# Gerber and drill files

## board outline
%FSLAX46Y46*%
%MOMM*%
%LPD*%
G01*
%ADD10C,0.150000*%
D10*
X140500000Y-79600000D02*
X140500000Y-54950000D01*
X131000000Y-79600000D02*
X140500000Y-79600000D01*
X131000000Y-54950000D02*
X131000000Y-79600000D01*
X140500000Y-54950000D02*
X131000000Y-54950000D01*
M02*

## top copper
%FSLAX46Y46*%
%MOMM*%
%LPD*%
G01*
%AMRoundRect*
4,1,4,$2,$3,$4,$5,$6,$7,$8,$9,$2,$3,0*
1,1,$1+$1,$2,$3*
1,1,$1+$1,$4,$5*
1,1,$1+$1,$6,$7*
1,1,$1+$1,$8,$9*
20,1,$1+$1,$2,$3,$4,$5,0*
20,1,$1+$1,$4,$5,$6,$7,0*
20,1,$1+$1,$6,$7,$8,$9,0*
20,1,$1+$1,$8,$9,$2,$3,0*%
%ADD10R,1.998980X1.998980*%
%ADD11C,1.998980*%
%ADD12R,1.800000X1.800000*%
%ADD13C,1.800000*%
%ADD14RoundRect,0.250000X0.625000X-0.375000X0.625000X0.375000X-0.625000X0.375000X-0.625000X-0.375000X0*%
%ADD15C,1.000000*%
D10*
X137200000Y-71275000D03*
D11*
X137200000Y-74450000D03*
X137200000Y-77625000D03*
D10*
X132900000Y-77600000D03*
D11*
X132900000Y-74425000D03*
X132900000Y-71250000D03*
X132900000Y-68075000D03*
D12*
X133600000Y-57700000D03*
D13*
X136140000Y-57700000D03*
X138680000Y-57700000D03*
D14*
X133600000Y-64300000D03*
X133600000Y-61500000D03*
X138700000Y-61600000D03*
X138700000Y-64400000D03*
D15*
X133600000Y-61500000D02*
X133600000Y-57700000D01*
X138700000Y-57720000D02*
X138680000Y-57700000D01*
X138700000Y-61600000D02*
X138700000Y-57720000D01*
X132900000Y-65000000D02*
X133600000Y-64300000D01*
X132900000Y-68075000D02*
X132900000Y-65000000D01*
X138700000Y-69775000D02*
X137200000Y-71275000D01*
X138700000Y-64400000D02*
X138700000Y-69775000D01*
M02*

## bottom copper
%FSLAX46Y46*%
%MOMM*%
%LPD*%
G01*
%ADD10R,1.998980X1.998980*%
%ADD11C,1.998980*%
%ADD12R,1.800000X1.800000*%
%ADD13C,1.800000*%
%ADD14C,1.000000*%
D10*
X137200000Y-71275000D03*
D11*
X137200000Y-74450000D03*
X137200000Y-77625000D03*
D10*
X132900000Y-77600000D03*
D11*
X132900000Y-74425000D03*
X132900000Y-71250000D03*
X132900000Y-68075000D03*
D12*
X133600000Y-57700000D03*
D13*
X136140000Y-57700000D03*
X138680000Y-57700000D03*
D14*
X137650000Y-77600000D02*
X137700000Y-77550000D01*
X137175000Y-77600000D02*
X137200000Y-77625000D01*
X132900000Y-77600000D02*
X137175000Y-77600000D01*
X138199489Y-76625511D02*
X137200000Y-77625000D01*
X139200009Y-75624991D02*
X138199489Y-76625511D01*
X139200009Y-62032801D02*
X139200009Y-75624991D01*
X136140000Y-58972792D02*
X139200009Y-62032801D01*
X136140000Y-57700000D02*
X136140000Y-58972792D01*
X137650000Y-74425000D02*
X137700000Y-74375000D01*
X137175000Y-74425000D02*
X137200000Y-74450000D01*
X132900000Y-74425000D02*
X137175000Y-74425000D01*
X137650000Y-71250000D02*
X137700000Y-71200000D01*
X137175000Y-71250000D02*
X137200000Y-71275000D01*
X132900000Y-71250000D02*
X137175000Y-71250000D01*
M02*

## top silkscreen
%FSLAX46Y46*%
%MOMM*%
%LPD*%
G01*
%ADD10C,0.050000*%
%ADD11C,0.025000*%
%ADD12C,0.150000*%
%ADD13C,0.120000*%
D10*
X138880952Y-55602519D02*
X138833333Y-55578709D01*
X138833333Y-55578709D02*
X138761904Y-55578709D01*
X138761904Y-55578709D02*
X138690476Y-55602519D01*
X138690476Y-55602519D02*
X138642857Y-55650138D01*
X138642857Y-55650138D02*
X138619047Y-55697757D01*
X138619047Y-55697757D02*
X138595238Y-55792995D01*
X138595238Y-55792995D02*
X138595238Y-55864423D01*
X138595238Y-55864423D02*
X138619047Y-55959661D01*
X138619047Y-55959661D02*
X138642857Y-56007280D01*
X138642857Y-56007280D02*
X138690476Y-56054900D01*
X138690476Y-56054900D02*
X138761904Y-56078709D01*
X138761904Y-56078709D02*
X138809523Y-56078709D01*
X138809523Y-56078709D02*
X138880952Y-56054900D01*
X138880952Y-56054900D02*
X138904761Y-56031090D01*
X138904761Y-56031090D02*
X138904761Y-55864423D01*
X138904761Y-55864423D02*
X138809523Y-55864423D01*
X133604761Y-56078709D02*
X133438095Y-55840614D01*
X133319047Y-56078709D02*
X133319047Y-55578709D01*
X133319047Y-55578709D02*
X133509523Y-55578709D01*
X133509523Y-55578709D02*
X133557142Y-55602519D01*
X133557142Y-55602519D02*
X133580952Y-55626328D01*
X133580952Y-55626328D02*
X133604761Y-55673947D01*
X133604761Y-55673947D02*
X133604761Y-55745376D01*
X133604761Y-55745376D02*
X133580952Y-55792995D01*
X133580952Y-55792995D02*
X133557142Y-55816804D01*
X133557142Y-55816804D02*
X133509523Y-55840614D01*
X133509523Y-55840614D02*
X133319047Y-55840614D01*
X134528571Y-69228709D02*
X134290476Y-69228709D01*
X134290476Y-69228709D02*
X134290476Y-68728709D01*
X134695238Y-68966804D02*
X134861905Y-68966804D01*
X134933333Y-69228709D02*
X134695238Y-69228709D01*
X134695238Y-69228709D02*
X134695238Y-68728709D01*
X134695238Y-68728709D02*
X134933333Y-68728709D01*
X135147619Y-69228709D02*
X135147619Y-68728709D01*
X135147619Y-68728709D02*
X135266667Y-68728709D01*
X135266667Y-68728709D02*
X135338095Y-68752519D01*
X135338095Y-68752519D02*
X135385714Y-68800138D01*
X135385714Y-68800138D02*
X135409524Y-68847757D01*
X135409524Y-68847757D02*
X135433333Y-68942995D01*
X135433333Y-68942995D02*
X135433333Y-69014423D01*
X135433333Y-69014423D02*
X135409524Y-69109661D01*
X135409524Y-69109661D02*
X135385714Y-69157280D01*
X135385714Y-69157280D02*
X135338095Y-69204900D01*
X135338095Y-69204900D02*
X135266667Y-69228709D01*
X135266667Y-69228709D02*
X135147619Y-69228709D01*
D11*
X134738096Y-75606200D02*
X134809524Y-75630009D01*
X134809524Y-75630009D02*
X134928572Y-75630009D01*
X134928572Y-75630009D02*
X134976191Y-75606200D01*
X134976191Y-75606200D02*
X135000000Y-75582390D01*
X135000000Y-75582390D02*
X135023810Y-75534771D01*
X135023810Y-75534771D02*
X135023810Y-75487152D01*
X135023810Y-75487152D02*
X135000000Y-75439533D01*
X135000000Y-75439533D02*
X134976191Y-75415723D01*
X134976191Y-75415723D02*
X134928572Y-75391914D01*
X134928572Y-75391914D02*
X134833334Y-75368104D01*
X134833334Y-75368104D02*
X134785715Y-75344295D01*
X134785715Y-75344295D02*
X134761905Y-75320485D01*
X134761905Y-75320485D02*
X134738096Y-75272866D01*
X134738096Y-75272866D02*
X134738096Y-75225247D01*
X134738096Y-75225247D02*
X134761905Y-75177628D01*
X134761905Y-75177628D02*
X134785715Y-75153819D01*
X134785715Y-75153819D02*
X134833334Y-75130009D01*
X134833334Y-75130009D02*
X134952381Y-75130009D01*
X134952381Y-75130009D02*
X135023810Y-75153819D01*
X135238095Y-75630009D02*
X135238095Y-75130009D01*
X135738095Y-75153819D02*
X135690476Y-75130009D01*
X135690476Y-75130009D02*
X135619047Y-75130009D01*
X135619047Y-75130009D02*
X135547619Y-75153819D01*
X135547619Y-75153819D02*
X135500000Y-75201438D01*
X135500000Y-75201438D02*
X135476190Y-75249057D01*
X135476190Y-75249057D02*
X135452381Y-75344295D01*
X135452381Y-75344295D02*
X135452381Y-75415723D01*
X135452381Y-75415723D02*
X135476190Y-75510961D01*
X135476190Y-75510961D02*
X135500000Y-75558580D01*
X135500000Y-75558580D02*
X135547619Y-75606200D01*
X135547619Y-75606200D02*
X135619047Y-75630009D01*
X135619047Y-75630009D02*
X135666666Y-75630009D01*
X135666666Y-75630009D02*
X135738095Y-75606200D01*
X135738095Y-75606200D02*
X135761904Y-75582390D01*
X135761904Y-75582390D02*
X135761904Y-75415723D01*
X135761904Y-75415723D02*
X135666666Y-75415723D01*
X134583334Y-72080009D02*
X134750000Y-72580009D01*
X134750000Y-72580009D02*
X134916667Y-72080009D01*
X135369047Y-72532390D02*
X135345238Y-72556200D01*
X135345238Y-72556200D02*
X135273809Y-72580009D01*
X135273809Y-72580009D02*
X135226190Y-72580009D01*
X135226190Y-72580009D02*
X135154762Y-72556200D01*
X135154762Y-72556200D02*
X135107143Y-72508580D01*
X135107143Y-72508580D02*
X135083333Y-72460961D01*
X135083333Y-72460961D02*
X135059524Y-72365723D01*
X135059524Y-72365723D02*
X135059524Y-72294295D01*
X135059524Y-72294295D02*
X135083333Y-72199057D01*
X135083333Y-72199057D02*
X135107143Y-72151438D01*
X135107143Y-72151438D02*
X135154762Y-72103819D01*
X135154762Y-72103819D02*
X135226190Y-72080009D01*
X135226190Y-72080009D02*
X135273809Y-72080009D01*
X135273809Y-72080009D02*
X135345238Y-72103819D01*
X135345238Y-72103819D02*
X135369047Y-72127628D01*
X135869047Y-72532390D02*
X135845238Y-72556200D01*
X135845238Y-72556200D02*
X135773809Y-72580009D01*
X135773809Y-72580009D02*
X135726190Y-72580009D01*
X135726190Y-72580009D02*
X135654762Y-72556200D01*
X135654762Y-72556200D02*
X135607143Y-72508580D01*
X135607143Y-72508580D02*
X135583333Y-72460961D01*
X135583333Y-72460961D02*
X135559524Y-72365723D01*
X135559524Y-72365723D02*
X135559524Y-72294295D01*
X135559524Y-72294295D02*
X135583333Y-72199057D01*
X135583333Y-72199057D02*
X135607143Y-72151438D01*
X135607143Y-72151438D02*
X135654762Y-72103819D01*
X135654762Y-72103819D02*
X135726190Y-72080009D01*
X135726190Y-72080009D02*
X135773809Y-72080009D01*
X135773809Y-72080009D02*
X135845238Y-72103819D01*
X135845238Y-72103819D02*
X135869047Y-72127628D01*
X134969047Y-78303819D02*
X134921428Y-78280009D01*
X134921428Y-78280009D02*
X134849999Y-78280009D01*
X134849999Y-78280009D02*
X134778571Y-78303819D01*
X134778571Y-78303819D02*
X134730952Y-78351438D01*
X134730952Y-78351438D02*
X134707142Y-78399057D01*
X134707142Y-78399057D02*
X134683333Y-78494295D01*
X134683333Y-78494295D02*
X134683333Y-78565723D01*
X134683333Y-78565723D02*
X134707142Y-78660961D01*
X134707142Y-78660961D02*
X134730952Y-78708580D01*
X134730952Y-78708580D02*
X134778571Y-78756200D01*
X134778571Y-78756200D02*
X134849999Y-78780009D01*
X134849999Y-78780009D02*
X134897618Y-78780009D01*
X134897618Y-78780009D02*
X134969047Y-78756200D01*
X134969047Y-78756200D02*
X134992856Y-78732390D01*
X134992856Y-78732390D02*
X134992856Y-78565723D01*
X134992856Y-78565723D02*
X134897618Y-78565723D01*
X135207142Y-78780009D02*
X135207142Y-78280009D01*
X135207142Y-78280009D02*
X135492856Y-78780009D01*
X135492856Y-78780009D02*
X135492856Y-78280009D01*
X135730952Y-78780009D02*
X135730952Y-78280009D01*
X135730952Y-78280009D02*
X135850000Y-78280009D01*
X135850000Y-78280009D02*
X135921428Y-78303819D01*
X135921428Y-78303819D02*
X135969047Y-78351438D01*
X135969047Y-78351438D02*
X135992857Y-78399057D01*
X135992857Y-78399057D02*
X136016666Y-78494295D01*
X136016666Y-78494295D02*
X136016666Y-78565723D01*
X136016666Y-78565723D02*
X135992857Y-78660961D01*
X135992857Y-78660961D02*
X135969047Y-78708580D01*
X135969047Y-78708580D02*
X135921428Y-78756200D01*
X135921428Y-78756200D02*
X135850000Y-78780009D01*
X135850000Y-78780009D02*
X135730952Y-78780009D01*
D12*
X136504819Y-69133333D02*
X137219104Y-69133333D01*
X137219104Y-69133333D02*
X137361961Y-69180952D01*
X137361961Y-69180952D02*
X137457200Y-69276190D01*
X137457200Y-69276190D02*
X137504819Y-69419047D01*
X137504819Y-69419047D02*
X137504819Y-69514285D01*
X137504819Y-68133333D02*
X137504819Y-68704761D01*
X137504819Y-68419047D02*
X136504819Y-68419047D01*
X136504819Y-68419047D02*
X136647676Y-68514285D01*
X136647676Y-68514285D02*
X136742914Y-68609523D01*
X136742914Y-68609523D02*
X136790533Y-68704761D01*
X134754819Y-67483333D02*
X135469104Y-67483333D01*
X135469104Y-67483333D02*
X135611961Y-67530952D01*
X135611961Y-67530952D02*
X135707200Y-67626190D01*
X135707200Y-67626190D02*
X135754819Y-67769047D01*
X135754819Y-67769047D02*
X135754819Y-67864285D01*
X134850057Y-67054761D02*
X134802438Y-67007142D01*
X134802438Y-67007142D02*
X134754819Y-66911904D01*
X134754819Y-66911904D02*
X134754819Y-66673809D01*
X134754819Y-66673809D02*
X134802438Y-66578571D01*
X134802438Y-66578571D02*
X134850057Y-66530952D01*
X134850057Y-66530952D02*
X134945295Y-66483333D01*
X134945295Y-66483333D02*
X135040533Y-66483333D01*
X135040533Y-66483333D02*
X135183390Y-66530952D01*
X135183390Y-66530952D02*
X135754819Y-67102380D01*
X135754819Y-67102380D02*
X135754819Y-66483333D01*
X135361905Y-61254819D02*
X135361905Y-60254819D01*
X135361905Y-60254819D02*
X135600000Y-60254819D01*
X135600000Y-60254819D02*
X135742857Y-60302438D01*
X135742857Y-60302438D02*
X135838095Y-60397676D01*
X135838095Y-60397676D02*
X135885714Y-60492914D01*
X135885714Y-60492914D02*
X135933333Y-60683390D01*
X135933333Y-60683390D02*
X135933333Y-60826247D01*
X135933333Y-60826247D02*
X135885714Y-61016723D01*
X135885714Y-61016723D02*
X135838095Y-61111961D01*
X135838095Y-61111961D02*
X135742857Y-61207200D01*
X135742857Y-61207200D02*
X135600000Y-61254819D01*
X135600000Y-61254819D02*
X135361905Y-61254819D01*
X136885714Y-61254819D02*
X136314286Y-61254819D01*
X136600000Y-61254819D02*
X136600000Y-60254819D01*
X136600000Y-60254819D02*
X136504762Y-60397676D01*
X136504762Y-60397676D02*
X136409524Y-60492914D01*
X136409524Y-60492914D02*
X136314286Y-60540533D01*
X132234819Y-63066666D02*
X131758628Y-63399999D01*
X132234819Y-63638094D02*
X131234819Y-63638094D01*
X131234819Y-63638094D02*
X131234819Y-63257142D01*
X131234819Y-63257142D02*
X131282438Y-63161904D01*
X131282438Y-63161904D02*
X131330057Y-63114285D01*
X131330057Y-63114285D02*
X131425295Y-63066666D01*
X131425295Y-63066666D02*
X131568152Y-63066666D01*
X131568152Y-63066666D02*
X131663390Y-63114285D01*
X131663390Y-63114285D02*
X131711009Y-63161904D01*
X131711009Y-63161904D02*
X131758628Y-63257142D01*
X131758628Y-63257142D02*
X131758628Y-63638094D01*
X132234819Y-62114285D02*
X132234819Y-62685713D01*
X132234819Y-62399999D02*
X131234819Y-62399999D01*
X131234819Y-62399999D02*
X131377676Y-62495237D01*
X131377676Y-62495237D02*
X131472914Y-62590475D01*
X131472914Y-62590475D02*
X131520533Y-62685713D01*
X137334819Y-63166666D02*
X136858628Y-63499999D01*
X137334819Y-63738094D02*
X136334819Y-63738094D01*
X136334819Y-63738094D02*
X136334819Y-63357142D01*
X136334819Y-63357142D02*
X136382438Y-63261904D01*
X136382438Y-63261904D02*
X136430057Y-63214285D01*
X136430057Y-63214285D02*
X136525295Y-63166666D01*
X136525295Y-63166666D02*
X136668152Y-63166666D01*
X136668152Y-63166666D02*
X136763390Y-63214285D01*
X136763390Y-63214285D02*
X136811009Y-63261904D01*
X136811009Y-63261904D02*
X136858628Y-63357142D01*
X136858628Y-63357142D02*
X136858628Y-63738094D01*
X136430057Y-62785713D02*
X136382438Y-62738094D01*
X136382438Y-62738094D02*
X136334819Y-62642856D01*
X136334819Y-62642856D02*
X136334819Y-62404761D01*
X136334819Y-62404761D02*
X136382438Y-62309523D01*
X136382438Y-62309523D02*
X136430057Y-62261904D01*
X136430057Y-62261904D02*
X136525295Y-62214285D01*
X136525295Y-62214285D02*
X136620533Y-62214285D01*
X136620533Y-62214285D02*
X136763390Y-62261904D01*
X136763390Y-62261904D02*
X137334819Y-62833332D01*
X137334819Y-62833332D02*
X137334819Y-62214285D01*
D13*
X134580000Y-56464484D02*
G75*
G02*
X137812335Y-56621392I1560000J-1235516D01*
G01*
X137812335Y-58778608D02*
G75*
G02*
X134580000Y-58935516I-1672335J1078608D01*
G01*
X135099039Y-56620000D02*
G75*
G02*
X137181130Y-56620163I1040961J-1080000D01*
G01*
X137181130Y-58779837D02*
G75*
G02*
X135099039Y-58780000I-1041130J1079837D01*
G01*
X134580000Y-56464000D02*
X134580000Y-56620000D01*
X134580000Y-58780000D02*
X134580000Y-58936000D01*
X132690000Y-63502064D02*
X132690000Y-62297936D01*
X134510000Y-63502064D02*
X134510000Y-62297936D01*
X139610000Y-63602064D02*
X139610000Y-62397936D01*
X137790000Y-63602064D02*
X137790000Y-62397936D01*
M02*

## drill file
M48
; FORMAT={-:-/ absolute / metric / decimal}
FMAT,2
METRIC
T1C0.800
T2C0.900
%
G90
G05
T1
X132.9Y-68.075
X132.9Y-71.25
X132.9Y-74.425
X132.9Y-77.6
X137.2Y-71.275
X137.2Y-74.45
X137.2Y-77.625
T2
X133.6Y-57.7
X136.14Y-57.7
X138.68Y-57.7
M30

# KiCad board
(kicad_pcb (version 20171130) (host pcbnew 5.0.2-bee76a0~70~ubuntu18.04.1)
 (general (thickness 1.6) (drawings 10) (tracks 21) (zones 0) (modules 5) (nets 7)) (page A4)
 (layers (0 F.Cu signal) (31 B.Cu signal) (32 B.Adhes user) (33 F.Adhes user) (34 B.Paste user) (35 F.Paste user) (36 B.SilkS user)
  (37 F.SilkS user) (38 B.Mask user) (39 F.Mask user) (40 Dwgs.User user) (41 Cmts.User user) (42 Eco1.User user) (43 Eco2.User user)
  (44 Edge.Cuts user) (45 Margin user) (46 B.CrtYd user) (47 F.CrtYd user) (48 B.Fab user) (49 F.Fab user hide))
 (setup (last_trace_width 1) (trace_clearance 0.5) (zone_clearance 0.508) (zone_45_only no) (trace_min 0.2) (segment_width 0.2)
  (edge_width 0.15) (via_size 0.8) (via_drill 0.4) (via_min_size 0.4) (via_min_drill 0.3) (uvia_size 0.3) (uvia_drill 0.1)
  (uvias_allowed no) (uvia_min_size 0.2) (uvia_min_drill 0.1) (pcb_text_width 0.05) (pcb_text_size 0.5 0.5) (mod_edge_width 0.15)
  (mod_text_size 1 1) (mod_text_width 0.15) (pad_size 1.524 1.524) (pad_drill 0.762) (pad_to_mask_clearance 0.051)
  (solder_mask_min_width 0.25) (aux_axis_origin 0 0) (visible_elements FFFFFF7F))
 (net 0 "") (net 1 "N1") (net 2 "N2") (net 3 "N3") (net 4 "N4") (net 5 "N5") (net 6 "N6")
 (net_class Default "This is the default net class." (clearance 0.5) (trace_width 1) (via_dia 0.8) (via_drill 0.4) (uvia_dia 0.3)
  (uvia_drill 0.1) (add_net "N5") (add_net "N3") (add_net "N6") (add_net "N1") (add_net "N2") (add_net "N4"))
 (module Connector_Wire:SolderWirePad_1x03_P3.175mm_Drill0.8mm (layer F.Cu) (at 137.2 71.275 270)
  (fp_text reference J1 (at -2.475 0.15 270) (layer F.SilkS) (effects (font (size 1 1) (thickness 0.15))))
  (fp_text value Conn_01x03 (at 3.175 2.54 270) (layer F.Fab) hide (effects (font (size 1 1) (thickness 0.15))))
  (pad 1 thru_hole rect (at 0 0 270) (size 1.99898 1.99898) (drill 0.8001) (layers *.Cu *.Mask) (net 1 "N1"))
  (pad 2 thru_hole circle (at 3.175 0 270) (size 1.99898 1.99898) (drill 0.8001) (layers *.Cu *.Mask) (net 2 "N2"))
  (pad 3 thru_hole circle (at 6.35 0 270) (size 1.99898 1.99898) (drill 0.8001) (layers *.Cu *.Mask) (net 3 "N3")))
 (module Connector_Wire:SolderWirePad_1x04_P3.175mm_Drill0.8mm (layer F.Cu) (at 132.9 77.6 90)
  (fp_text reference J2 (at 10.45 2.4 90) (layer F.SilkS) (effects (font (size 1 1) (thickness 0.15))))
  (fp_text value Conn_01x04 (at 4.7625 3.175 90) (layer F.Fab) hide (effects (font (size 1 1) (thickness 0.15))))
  (pad 1 thru_hole rect (at 0 0 90) (size 1.99898 1.99898) (drill 0.8001) (layers *.Cu *.Mask) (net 3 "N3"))
  (pad 2 thru_hole circle (at 3.175 0 90) (size 1.99898 1.99898) (drill 0.8001) (layers *.Cu *.Mask) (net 2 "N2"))
  (pad 3 thru_hole circle (at 6.35 0 90) (size 1.99898 1.99898) (drill 0.8001) (layers *.Cu *.Mask) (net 1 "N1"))
  (pad 4 thru_hole circle (at 9.525 0 90) (size 1.99898 1.99898) (drill 0.8001) (layers *.Cu *.Mask) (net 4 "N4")))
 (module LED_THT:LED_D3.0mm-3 (layer F.Cu) (at 133.6 57.7)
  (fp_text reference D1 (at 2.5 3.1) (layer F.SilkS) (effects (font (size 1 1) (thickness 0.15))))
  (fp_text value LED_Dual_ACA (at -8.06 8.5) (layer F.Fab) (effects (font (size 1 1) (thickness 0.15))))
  (fp_arc (start 2.54 0) (end 0.98 -1.235516) (angle 108.8) (layer F.SilkS) (width 0.12))
  (fp_arc (start 2.54 0) (end 0.98 1.235516) (angle -108.8) (layer F.SilkS) (width 0.12))
  (fp_arc (start 2.54 0) (end 1.499039 -1.08) (angle 87.9) (layer F.SilkS) (width 0.12))
  (fp_arc (start 2.54 0) (end 1.499039 1.08) (angle -87.9) (layer F.SilkS) (width 0.12))
  (fp_line (start 0.98 -1.236) (end 0.98 -1.08) (layer F.SilkS) (width 0.12))
  (fp_line (start 0.98 1.08) (end 0.98 1.236) (layer F.SilkS) (width 0.12))
  (pad 1 thru_hole rect (at 0 0) (size 1.8 1.8) (drill 0.9) (layers *.Cu *.Mask) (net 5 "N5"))
  (pad 2 thru_hole circle (at 2.54 0) (size 1.8 1.8) (drill 0.9) (layers *.Cu *.Mask) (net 3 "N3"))
  (pad 3 thru_hole circle (at 5.08 0) (size 1.8 1.8) (drill 0.9) (layers *.Cu *.Mask) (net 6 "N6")))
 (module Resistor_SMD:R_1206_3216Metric (layer F.Cu) (at 133.6 62.9 90)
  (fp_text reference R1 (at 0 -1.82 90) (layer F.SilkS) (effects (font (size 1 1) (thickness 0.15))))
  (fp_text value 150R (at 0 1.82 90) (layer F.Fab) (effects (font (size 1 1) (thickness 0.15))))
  (fp_line (start -0.602064 -0.91) (end 0.602064 -0.91) (layer F.SilkS) (width 0.12))
  (fp_line (start -0.602064 0.91) (end 0.602064 0.91) (layer F.SilkS) (width 0.12))
  (pad 1 smd roundrect (at -1.4 0 90) (size 1.25 1.75) (layers F.Cu F.Paste F.Mask) (roundrect_rratio 0.2) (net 4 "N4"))
  (pad 2 smd roundrect (at 1.4 0 90) (size 1.25 1.75) (layers F.Cu F.Paste F.Mask) (roundrect_rratio 0.2) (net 5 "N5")))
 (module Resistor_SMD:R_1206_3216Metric (layer F.Cu) (at 138.7 63 90)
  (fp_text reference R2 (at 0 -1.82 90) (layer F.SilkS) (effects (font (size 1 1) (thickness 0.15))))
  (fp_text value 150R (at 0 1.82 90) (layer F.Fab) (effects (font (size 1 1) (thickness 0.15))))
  (fp_line (start -0.602064 0.91) (end 0.602064 0.91) (layer F.SilkS) (width 0.12))
  (fp_line (start -0.602064 -0.91) (end 0.602064 -0.91) (layer F.SilkS) (width 0.12))
  (pad 2 smd roundrect (at 1.4 0 90) (size 1.25 1.75) (layers F.Cu F.Paste F.Mask) (roundrect_rratio 0.2) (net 6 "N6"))
  (pad 1 smd roundrect (at -1.4 0 90) (size 1.25 1.75) (layers F.Cu F.Paste F.Mask) (roundrect_rratio 0.2) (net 1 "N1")))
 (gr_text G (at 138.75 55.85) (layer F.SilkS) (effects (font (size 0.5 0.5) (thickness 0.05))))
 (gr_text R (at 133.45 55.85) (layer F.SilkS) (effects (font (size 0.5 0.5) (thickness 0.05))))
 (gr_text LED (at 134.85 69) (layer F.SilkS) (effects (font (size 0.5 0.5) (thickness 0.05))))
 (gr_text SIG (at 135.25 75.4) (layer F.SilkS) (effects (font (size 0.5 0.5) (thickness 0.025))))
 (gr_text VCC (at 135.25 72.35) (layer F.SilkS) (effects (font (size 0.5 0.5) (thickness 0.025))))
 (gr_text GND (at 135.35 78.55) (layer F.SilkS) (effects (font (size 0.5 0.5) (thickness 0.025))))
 (gr_line (start 140.5 79.6) (end 140.5 54.95) (layer Edge.Cuts) (width 0.15))
 (gr_line (start 131 79.6) (end 140.5 79.6) (layer Edge.Cuts) (width 0.15))
 (gr_line (start 131 54.95) (end 131 79.6) (layer Edge.Cuts) (width 0.15))
 (gr_line (start 140.5 54.95) (end 131 54.95) (layer Edge.Cuts) (width 0.15))
 (segment (start 133.6 61.5) (end 133.6 57.7) (width 1) (layer F.Cu) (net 5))
 (segment (start 137.65 77.6) (end 137.7 77.55) (width 1) (layer B.Cu) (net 3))
 (segment (start 137.175 77.6) (end 137.2 77.625) (width 1) (layer B.Cu) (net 3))
 (segment (start 132.9 77.6) (end 137.175 77.6) (width 1) (layer B.Cu) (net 3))
 (segment (start 138.199489 76.625511) (end 137.2 77.625) (width 1) (layer B.Cu) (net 3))
 (segment (start 139.200009 75.624991) (end 138.199489 76.625511) (width 1) (layer B.Cu) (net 3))
 (segment (start 139.200009 62.032801) (end 139.200009 75.624991) (width 1) (layer B.Cu) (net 3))
 (segment (start 136.14 58.972792) (end 139.200009 62.032801) (width 1) (layer B.Cu) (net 3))
 (segment (start 136.14 57.7) (end 136.14 58.972792) (width 1) (layer B.Cu) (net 3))
 (segment (start 137.65 74.425) (end 137.7 74.375) (width 1) (layer B.Cu) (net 2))
 (segment (start 137.175 74.425) (end 137.2 74.45) (width 1) (layer B.Cu) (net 2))
 (segment (start 132.9 74.425) (end 137.175 74.425) (width 1) (layer B.Cu) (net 2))
 (segment (start 138.7 57.72) (end 138.68 57.7) (width 1) (layer F.Cu) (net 6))
 (segment (start 138.7 61.6) (end 138.7 57.72) (width 1) (layer F.Cu) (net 6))
 (segment (start 132.9 65) (end 133.6 64.3) (width 1) (layer F.Cu) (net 4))
 (segment (start 132.9 68.075) (end 132.9 65) (width 1) (layer F.Cu) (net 4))
 (segment (start 137.65 71.25) (end 137.7 71.2) (width 1) (layer B.Cu) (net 1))
 (segment (start 137.175 71.25) (end 137.2 71.275) (width 1) (layer B.Cu) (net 1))
 (segment (start 132.9 71.25) (end 137.175 71.25) (width 1) (layer B.Cu) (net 1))
 (segment (start 138.7 69.775) (end 137.2 71.275) (width 1) (layer F.Cu) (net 1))
 (segment (start 138.7 64.4) (end 138.7 69.775) (width 1) (layer F.Cu) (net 1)))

